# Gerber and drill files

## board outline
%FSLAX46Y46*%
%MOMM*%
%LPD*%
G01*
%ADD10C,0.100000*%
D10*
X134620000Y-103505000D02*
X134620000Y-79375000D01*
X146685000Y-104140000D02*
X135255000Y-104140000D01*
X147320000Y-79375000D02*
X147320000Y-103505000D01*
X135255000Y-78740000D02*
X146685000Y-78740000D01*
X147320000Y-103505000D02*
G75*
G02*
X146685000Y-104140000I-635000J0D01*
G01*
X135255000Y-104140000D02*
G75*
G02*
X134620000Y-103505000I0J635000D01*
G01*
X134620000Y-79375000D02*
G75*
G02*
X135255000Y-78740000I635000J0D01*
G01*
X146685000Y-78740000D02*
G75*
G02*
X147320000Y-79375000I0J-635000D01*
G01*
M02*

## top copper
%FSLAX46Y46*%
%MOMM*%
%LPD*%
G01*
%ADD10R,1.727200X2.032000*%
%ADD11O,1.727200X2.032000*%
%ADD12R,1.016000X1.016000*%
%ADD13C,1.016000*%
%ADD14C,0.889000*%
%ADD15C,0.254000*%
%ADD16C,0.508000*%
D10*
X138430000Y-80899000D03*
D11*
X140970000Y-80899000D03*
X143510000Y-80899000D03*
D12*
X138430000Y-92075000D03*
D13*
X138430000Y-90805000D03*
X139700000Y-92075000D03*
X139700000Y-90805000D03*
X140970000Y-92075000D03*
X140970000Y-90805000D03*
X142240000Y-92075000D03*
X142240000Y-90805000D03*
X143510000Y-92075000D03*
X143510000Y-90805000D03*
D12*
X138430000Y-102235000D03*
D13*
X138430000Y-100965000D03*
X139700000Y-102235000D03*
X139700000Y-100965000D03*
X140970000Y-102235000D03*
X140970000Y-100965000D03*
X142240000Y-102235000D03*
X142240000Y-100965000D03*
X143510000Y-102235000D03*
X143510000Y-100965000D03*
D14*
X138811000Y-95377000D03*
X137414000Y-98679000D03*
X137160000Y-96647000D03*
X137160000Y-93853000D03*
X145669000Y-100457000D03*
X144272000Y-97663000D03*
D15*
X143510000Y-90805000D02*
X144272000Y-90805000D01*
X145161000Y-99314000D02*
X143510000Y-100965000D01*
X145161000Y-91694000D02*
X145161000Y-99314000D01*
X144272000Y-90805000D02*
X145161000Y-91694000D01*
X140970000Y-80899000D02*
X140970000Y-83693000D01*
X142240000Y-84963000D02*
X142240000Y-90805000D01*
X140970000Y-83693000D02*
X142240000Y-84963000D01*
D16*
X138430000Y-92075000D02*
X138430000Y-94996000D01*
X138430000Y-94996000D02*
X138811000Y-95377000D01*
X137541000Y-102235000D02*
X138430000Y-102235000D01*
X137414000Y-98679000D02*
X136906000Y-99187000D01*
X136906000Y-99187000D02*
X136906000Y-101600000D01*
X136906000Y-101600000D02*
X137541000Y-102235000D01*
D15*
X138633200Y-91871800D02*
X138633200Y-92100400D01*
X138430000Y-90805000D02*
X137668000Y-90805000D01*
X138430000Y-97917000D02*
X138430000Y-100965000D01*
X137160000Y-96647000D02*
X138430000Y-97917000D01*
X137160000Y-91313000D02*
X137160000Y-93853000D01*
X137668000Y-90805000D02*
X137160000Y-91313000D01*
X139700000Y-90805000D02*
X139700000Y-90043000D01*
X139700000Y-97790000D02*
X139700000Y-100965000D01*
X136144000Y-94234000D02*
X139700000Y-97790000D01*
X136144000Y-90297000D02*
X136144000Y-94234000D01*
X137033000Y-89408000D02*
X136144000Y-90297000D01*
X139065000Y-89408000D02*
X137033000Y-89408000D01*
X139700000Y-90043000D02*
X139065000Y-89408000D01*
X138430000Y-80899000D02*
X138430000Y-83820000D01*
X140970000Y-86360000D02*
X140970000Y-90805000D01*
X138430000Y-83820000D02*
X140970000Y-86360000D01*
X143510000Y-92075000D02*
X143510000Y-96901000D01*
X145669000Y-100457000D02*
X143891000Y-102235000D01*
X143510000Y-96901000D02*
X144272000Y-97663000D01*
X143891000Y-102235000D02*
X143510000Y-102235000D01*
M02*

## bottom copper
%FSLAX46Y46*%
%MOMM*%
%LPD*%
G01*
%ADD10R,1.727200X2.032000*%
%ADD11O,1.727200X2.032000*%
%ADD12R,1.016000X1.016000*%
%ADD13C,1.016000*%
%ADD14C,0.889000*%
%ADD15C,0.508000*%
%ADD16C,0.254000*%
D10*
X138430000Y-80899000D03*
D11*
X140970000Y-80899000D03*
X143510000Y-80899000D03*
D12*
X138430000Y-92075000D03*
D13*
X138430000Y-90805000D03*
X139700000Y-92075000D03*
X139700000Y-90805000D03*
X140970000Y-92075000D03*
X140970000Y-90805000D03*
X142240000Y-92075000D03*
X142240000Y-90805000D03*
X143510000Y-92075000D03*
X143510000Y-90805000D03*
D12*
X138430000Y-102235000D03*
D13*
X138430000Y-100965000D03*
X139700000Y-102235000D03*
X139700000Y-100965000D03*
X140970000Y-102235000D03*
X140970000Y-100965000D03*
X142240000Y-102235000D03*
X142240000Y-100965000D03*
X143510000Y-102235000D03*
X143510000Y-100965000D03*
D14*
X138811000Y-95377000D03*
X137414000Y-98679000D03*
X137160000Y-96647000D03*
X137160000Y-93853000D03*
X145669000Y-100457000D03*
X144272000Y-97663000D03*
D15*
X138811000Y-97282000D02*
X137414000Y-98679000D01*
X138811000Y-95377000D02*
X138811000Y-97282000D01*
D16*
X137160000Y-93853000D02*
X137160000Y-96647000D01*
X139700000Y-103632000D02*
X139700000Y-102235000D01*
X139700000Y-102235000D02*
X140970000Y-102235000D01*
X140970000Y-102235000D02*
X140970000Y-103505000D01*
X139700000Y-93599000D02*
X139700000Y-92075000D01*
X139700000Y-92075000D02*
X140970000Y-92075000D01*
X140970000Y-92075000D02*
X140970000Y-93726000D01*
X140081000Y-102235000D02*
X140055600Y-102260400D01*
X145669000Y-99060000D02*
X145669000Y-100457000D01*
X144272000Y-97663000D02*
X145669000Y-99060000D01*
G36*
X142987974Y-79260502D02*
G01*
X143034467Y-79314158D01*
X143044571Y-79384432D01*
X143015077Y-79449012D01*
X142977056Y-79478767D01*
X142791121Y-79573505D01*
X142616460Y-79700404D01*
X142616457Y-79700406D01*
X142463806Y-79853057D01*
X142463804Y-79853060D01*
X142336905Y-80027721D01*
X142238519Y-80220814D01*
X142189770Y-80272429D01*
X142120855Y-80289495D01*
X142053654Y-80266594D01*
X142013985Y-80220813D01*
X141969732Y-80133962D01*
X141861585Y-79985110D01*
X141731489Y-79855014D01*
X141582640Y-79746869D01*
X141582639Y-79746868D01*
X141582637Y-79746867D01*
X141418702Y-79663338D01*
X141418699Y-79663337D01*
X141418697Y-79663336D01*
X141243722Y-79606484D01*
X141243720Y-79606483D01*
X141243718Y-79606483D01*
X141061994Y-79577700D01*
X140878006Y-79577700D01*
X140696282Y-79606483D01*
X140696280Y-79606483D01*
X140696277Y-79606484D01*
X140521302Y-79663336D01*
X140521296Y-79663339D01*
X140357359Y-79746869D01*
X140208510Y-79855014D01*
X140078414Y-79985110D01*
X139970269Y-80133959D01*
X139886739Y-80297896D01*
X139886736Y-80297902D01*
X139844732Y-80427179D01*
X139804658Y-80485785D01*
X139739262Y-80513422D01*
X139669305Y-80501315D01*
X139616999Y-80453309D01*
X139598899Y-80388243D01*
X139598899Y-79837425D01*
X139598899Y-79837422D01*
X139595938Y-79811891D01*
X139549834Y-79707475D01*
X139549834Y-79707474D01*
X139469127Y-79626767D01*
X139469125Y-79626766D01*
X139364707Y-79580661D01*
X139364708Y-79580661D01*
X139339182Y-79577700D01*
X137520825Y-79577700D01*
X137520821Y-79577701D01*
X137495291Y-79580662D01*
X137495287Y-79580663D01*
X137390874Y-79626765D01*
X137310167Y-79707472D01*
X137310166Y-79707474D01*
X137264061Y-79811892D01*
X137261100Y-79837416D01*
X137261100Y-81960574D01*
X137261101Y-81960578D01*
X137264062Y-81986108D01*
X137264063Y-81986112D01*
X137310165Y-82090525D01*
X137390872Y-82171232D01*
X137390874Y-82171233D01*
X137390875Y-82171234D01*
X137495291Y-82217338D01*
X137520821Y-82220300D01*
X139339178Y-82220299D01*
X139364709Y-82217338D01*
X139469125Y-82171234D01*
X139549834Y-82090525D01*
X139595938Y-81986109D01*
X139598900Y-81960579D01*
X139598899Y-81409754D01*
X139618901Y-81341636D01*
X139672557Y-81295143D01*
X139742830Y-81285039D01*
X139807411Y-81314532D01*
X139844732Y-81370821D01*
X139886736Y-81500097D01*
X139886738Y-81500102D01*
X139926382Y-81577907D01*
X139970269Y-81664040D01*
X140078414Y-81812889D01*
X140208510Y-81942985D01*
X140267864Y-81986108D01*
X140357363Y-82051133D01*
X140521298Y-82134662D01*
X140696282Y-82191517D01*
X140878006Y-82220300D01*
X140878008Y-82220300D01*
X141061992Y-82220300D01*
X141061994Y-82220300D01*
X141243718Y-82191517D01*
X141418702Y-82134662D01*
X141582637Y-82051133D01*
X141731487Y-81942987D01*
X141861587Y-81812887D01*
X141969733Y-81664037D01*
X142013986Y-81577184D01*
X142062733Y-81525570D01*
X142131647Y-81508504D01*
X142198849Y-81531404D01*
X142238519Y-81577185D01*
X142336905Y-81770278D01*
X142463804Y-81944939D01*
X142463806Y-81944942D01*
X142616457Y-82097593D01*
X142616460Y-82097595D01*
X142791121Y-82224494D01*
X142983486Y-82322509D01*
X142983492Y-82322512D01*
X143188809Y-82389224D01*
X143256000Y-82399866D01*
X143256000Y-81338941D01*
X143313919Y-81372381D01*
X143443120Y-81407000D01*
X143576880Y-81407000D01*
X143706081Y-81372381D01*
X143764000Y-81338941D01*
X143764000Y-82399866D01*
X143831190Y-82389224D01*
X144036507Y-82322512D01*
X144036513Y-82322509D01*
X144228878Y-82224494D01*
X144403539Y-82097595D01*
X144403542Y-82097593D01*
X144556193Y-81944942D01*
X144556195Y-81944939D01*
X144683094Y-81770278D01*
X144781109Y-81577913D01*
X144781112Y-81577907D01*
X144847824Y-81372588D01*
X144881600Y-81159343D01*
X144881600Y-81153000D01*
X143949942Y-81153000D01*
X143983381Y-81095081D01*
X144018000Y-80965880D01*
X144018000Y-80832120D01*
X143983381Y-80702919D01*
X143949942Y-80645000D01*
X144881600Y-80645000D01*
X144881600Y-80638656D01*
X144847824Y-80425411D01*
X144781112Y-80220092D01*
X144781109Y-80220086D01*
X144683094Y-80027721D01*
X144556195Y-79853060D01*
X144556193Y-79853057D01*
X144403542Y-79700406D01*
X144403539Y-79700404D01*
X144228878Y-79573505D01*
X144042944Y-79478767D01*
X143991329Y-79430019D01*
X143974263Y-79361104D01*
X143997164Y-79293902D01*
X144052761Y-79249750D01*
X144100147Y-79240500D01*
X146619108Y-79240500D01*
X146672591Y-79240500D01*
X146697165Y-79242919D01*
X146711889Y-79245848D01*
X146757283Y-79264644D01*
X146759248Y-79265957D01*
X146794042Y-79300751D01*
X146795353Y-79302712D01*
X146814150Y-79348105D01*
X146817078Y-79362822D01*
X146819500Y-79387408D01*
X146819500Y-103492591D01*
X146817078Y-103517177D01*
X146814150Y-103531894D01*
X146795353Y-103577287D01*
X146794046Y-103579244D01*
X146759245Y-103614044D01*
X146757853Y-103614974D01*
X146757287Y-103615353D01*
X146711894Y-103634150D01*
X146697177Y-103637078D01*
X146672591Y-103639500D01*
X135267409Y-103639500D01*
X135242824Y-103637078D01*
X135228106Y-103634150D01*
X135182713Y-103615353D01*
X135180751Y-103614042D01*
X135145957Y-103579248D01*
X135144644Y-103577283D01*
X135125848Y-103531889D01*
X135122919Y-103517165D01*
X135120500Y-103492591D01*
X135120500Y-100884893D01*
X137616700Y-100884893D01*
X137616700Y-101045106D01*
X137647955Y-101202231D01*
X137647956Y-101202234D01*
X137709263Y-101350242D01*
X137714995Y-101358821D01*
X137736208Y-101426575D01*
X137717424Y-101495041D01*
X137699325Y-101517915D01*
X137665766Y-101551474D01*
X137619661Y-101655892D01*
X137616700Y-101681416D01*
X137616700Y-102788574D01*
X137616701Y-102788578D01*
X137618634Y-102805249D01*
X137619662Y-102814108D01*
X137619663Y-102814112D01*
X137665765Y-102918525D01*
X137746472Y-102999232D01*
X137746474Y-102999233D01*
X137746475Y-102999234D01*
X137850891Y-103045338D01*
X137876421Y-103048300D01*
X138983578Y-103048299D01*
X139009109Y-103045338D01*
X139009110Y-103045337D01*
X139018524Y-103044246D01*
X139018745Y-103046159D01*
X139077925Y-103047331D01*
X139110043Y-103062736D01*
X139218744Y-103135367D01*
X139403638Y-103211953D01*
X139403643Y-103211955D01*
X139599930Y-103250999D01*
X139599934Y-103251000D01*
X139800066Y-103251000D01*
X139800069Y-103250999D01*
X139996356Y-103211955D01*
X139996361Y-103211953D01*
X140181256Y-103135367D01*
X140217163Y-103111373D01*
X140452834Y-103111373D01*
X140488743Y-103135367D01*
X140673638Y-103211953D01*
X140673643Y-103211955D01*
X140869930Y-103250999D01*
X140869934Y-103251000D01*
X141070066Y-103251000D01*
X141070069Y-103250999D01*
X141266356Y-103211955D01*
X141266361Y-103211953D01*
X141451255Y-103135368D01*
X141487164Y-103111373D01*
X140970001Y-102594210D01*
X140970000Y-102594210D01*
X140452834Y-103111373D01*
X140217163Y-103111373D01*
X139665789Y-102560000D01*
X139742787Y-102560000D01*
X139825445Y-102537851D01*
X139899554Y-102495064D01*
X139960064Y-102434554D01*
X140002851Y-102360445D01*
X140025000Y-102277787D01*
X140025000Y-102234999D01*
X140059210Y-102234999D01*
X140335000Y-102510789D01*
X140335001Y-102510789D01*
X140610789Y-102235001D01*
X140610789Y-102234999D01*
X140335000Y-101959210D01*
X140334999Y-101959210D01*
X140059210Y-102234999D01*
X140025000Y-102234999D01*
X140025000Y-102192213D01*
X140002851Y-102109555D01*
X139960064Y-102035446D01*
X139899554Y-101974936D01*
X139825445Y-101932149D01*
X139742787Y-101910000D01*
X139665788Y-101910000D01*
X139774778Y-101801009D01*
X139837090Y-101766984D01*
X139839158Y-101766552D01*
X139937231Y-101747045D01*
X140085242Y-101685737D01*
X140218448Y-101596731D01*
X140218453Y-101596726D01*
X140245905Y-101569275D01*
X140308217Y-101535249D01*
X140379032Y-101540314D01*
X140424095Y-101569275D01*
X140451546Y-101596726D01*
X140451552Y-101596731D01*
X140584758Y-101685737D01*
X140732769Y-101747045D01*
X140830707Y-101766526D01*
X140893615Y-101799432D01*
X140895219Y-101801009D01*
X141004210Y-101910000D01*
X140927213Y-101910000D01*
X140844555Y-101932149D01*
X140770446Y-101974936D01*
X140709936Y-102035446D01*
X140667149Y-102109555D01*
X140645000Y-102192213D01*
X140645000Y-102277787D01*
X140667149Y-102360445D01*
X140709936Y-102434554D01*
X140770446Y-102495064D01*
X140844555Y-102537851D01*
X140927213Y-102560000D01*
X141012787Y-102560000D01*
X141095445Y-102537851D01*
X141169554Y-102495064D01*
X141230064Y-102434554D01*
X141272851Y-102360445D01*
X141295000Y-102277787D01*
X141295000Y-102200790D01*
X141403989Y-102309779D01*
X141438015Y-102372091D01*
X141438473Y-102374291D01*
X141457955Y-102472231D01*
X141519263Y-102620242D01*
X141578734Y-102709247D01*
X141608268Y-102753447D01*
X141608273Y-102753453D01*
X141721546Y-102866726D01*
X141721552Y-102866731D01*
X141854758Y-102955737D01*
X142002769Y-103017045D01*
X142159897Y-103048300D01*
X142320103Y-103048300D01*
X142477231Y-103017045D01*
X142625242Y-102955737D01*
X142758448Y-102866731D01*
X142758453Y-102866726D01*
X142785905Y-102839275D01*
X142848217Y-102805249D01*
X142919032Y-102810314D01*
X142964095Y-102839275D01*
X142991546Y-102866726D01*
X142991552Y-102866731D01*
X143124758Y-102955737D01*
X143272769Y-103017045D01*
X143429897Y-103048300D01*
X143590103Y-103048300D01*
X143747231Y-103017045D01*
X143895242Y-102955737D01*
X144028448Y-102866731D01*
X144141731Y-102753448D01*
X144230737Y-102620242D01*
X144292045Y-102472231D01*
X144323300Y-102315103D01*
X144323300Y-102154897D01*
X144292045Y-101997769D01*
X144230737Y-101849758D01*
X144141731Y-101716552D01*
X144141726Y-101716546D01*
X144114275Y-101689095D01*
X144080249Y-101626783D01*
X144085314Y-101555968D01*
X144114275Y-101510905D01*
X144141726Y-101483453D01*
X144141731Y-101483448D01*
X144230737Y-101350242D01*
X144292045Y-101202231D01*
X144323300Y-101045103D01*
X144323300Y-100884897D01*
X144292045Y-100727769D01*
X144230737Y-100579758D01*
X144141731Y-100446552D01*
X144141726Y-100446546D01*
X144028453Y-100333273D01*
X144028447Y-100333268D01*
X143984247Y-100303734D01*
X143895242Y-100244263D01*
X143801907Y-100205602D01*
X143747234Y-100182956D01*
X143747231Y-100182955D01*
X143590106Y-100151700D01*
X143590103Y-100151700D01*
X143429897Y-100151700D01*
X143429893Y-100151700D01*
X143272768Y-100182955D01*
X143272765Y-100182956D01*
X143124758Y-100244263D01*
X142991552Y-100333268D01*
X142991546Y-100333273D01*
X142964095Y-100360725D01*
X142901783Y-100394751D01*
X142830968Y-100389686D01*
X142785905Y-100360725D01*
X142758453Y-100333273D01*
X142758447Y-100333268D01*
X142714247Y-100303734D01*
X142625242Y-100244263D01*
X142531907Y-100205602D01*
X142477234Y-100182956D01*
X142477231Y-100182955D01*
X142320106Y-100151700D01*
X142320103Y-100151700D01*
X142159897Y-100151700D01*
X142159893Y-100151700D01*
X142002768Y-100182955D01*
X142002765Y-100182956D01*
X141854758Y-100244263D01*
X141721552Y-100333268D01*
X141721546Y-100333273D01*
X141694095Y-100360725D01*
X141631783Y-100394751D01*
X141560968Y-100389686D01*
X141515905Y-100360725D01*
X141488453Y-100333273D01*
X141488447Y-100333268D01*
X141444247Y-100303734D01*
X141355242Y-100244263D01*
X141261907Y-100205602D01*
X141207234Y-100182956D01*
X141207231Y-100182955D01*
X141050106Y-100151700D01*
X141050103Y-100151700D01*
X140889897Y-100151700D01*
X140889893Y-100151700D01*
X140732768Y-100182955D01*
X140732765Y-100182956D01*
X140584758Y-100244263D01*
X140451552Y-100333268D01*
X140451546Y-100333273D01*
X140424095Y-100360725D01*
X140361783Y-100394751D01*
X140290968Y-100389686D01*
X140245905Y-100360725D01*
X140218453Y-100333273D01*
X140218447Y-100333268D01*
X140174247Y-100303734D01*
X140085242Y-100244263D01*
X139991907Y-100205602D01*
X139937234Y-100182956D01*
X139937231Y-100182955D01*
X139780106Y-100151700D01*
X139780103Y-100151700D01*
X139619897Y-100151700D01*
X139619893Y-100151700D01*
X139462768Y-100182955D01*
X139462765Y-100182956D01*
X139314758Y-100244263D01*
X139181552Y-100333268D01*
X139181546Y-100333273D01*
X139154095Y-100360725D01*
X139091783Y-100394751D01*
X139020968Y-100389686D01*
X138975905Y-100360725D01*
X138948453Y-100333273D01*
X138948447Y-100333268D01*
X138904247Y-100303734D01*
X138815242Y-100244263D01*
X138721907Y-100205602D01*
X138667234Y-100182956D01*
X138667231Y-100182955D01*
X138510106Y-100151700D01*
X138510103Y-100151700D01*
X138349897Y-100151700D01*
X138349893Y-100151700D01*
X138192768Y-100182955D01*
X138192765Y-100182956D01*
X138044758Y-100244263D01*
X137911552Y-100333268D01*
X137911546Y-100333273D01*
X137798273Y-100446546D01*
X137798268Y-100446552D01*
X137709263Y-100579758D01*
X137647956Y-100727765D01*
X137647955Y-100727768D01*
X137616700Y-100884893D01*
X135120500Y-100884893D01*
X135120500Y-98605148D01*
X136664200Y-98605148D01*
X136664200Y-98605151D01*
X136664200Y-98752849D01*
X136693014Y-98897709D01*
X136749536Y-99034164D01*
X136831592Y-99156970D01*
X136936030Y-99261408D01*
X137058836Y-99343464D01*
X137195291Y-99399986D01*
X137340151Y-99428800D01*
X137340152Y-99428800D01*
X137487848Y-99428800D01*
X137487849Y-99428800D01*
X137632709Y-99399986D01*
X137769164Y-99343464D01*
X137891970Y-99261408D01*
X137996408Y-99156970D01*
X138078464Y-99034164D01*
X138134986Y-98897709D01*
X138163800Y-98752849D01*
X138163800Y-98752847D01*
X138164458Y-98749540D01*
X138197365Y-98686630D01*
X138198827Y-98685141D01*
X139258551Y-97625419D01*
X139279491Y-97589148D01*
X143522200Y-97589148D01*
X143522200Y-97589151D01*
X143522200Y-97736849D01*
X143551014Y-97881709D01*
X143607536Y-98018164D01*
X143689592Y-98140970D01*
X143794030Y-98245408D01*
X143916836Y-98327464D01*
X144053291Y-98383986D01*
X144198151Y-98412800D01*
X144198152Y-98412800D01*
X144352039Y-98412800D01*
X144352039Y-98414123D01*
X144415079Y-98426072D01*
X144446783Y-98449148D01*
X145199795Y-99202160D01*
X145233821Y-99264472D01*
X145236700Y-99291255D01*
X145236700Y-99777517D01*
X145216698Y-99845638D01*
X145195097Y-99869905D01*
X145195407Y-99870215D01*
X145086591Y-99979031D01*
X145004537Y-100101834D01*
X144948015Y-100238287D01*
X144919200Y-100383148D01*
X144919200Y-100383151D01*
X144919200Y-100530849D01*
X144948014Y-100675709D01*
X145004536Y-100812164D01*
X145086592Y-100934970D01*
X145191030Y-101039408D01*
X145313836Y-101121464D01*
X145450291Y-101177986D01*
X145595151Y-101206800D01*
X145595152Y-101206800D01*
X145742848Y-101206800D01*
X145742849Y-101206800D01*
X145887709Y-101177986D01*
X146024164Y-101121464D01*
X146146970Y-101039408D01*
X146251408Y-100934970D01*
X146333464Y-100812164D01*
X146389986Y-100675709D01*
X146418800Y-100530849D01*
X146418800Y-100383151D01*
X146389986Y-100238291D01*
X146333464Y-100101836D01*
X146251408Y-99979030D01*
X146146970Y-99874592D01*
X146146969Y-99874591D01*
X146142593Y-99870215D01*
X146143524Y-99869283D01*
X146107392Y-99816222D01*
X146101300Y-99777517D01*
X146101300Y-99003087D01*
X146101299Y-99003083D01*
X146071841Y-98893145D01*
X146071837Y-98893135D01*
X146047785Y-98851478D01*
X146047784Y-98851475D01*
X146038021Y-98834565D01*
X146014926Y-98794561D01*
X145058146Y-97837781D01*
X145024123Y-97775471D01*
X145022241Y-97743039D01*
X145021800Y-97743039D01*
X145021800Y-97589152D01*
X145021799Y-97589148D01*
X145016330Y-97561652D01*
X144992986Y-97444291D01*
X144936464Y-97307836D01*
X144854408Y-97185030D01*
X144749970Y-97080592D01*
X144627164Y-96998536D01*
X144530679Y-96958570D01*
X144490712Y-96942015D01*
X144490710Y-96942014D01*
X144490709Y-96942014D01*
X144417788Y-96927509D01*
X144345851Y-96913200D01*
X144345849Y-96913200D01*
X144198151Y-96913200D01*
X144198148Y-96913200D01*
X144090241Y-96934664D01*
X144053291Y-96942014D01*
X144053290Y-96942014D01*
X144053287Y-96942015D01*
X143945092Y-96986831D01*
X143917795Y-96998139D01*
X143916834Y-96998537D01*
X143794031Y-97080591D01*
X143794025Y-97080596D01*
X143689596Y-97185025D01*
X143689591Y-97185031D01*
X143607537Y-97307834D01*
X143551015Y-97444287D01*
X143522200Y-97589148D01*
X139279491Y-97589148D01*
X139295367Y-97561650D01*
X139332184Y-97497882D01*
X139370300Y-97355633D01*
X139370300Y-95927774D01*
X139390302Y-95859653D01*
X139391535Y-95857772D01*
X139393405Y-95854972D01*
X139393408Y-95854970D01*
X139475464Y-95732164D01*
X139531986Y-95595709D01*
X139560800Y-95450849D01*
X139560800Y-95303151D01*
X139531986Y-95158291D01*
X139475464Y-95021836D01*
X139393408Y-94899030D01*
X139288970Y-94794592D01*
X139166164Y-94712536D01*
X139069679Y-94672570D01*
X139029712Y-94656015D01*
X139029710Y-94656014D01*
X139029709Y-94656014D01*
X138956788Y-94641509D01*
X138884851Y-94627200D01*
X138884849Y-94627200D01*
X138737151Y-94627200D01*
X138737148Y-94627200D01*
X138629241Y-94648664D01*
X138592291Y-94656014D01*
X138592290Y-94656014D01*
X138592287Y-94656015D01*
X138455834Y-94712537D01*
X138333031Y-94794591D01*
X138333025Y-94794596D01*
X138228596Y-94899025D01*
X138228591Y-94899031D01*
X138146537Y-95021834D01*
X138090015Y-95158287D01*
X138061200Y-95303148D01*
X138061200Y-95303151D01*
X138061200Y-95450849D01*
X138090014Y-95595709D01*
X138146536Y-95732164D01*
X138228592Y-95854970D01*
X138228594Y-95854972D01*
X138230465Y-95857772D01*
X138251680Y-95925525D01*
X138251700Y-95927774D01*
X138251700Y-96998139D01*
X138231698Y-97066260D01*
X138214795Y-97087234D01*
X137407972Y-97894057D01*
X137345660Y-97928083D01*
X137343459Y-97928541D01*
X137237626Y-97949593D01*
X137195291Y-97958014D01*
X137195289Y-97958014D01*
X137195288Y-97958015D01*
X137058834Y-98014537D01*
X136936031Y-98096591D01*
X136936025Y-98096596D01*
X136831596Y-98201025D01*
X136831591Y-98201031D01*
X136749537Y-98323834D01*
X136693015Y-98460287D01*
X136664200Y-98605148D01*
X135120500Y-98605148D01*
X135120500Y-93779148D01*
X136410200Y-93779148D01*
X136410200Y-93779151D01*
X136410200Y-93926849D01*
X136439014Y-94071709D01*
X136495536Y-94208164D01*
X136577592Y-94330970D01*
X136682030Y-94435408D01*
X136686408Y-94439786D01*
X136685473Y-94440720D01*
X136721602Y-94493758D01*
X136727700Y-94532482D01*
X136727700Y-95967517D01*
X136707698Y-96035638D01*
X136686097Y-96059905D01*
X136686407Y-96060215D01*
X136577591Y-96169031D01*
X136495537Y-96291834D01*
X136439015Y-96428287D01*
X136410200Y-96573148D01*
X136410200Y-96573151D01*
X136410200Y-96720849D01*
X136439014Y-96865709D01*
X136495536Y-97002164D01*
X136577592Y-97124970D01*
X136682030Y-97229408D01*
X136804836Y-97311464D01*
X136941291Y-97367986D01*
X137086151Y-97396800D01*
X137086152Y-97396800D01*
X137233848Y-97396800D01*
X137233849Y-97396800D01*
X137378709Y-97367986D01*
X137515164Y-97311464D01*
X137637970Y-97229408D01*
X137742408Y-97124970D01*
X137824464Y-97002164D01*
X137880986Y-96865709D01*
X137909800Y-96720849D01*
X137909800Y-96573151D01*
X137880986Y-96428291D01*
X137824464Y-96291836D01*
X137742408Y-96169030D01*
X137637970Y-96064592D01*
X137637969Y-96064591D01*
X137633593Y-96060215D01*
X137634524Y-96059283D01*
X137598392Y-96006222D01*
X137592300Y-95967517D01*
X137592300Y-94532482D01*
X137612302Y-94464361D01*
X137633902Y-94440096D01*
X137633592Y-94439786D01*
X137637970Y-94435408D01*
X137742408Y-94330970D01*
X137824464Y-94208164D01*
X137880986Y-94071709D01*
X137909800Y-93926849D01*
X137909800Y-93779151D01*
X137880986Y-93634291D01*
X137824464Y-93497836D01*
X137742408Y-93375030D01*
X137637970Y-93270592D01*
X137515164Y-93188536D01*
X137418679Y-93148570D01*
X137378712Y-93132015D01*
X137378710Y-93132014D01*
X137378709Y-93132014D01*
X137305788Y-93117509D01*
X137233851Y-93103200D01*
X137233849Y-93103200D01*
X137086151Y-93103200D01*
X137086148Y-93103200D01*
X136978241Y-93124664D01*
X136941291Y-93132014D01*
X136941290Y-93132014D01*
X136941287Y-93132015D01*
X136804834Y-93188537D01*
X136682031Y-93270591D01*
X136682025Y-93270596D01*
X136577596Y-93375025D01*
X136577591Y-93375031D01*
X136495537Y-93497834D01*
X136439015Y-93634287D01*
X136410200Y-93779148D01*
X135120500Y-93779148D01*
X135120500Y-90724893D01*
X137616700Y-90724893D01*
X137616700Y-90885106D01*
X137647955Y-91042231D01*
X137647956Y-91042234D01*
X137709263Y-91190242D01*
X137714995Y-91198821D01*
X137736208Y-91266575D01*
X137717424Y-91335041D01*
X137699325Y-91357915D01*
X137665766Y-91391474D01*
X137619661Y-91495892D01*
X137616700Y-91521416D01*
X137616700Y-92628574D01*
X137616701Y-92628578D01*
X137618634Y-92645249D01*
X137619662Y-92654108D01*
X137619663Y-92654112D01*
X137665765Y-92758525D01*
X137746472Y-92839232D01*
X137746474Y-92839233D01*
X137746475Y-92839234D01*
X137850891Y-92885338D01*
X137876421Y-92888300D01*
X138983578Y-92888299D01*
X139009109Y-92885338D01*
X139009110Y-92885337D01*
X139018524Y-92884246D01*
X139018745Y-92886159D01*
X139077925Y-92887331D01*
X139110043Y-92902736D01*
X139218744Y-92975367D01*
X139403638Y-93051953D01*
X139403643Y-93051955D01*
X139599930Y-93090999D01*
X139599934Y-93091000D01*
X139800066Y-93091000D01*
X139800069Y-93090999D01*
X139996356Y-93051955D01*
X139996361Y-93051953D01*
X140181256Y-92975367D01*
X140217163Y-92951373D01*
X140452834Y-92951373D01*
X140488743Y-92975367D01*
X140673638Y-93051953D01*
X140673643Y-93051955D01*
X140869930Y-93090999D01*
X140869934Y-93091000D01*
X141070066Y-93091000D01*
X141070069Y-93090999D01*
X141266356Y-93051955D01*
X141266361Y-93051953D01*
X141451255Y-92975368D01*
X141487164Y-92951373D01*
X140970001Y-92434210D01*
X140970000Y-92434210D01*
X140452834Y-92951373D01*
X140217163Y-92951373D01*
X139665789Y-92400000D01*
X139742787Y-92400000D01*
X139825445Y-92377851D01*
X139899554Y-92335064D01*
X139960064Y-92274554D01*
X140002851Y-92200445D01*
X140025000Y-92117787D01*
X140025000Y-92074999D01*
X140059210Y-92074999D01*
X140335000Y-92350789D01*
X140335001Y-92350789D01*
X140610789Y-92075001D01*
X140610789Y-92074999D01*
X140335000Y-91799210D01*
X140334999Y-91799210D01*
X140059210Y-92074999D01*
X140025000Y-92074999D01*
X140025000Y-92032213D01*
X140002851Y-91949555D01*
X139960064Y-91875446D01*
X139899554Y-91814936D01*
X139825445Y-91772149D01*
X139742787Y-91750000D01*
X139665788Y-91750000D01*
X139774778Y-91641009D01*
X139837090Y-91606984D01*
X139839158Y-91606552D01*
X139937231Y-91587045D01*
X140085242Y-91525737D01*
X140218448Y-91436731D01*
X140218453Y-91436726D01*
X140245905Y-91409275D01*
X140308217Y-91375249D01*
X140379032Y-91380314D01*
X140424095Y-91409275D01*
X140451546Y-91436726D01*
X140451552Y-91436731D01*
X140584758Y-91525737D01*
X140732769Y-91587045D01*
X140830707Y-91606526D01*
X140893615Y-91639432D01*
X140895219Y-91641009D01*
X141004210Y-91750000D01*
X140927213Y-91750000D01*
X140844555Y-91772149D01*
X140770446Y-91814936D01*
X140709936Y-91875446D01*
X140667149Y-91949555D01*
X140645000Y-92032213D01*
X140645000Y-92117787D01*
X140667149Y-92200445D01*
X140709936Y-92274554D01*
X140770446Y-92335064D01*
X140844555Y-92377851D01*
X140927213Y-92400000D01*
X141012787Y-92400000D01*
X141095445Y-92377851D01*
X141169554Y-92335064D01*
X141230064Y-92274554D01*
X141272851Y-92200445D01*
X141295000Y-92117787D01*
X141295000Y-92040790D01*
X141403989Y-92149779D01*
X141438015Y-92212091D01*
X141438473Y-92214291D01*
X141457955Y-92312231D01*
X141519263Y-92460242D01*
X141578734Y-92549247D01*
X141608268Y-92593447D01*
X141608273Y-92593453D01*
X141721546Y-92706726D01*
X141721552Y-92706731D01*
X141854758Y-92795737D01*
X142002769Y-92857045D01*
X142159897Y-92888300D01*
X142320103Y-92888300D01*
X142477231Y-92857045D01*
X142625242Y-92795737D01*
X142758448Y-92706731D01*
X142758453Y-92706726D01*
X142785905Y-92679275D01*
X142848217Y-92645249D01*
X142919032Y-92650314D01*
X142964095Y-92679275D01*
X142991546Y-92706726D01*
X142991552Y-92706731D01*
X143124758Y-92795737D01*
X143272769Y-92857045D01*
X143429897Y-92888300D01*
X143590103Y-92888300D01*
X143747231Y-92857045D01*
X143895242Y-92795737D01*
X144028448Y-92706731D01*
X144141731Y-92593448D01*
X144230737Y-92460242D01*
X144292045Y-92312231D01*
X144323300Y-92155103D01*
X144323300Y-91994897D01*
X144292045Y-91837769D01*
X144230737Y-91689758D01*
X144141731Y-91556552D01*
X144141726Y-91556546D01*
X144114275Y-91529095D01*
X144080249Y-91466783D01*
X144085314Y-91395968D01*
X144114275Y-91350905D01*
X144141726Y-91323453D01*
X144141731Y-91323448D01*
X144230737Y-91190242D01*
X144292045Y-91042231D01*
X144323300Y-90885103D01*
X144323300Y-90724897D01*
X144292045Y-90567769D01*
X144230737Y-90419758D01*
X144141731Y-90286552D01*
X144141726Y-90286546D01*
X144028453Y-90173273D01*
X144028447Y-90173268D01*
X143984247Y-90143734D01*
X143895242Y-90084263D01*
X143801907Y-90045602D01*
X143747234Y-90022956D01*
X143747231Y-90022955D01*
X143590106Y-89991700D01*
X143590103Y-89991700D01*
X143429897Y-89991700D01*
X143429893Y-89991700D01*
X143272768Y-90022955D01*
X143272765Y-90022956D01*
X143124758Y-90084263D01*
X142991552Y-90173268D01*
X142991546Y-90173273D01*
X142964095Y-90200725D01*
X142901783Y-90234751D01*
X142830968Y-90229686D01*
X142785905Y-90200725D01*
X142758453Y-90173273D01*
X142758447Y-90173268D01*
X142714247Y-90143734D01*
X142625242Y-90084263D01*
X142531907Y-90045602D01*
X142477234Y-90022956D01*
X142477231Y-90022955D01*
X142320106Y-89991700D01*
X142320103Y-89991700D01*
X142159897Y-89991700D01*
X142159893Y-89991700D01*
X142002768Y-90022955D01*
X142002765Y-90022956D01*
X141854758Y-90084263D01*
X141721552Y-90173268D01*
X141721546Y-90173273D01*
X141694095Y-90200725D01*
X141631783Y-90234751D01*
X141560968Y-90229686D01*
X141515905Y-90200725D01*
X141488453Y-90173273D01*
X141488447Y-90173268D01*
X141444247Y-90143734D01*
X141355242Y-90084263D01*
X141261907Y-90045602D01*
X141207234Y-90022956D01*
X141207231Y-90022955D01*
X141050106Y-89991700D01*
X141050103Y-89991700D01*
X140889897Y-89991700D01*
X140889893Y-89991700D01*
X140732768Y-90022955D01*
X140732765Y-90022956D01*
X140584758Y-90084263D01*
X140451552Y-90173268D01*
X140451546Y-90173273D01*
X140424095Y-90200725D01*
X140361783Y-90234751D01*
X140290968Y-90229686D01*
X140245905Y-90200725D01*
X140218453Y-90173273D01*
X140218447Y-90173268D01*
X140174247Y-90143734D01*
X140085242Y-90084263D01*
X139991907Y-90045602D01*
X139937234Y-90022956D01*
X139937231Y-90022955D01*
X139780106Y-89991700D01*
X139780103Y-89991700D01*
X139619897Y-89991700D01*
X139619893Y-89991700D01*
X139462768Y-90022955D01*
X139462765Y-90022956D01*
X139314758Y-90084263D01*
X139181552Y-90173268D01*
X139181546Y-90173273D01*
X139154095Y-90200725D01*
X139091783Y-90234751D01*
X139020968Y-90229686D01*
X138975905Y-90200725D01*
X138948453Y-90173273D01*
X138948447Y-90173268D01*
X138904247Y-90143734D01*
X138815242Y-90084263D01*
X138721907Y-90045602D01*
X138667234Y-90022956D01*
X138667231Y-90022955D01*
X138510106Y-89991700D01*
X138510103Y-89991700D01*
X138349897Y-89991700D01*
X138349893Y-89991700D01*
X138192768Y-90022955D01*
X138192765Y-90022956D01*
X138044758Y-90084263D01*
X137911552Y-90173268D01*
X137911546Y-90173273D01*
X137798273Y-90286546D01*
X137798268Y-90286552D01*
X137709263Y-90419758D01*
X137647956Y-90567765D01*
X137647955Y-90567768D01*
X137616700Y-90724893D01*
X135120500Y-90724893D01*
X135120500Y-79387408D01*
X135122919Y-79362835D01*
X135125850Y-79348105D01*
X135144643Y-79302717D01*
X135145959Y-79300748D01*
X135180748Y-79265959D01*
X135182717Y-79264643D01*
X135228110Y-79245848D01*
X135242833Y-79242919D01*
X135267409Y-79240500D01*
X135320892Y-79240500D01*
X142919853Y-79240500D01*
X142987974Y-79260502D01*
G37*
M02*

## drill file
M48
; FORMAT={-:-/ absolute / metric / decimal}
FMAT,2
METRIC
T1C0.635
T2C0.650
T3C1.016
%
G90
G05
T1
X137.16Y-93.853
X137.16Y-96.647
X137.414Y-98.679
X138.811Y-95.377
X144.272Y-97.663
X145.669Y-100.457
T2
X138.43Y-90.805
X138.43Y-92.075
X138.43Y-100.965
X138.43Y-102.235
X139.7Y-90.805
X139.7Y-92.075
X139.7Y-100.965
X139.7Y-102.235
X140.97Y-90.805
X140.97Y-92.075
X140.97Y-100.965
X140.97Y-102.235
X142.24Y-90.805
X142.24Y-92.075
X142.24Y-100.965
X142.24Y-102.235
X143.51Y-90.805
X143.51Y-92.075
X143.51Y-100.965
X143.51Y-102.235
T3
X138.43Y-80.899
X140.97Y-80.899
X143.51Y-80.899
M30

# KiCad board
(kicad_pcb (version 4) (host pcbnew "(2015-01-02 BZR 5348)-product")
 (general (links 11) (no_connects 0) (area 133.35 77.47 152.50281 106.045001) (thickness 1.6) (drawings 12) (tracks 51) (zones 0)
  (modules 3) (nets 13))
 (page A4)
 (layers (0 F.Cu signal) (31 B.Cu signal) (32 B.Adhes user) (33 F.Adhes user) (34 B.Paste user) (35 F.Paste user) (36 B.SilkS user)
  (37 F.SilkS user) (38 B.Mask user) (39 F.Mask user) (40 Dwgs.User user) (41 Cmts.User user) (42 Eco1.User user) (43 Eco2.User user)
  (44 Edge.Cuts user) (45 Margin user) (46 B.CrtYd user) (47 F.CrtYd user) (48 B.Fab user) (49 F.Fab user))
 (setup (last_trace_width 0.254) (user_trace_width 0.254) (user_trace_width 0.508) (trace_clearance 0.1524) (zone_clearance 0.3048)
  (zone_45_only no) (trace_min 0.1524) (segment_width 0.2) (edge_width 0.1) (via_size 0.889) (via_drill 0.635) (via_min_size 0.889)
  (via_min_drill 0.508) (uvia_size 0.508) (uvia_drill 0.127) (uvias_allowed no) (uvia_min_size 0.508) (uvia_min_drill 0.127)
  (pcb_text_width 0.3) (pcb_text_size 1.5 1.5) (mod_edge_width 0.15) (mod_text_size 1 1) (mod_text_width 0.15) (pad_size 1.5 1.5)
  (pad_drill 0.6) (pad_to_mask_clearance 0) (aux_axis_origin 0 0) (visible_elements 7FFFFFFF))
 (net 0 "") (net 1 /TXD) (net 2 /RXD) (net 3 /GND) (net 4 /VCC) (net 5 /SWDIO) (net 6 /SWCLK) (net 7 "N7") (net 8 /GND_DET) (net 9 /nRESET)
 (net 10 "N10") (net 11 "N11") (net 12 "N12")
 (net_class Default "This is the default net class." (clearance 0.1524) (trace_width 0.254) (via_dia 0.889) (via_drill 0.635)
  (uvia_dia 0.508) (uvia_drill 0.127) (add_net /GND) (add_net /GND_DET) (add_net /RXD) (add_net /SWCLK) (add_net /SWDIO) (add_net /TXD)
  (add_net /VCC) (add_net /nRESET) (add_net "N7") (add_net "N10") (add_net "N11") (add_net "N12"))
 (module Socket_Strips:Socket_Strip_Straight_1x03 (layer F.Cu) (at 140.97 80.899 180)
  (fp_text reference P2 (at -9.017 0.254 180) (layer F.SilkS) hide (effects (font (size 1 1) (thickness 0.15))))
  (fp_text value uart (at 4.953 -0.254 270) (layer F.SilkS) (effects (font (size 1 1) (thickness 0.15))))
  (pad 1 thru_hole rect (at 2.54 0) (size 1.7272 2.032) (drill 1.016) (layers *.Cu *.Mask F.SilkS) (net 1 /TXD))
  (pad 2 thru_hole oval (at 0 0) (size 1.7272 2.032) (drill 1.016) (layers *.Cu *.Mask F.SilkS) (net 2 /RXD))
  (pad 3 thru_hole oval (at -2.54 0) (size 1.7272 2.032) (drill 1.016) (layers *.Cu *.Mask F.SilkS) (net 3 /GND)))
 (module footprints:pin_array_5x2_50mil (layer F.Cu) (at 139.7 91.44)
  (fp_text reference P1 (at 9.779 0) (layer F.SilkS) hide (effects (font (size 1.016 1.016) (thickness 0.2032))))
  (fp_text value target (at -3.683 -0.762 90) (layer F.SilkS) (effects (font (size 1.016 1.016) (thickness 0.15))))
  (pad 1 thru_hole rect (at -1.27 0.635) (size 1.016 1.016) (drill 0.65) (layers *.Cu *.Mask F.SilkS) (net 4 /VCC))
  (pad 2 thru_hole circle (at -1.27 -0.635) (size 1.016 1.016) (drill 0.65) (layers *.Cu *.Mask F.SilkS) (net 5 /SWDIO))
  (pad 3 thru_hole circle (at 0 0.635) (size 1.016 1.016) (drill 0.65) (layers *.Cu *.Mask F.SilkS) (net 3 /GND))
  (pad 4 thru_hole circle (at 0 -0.635) (size 1.016 1.016) (drill 0.65) (layers *.Cu *.Mask F.SilkS) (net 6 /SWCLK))
  (pad 5 thru_hole circle (at 1.27 0.635) (size 1.016 1.016) (drill 0.65) (layers *.Cu *.Mask F.SilkS) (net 3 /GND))
  (pad 6 thru_hole circle (at 1.27 -0.635) (size 1.016 1.016) (drill 0.65) (layers *.Cu *.Mask F.SilkS) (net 1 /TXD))
  (pad 7 thru_hole circle (at 2.54 0.635) (size 1.016 1.016) (drill 0.65) (layers *.Cu *.Mask F.SilkS) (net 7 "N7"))
  (pad 8 thru_hole circle (at 2.54 -0.635) (size 1.016 1.016) (drill 0.65) (layers *.Cu *.Mask F.SilkS) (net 2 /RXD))
  (pad 9 thru_hole circle (at 3.81 0.635) (size 1.016 1.016) (drill 0.65) (layers *.Cu *.Mask F.SilkS) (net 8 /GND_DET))
  (pad 10 thru_hole circle (at 3.81 -0.635) (size 1.016 1.016) (drill 0.65) (layers *.Cu *.Mask F.SilkS) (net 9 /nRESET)))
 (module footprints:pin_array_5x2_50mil (layer F.Cu) (at 139.7 101.6)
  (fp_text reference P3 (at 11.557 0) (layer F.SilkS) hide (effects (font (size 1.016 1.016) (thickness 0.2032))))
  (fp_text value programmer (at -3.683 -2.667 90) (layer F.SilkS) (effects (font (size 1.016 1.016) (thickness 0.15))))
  (pad 1 thru_hole rect (at -1.27 0.635) (size 1.016 1.016) (drill 0.65) (layers *.Cu *.Mask F.SilkS) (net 4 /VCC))
  (pad 2 thru_hole circle (at -1.27 -0.635) (size 1.016 1.016) (drill 0.65) (layers *.Cu *.Mask F.SilkS) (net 5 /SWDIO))
  (pad 3 thru_hole circle (at 0 0.635) (size 1.016 1.016) (drill 0.65) (layers *.Cu *.Mask F.SilkS) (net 3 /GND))
  (pad 4 thru_hole circle (at 0 -0.635) (size 1.016 1.016) (drill 0.65) (layers *.Cu *.Mask F.SilkS) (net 6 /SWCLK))
  (pad 5 thru_hole circle (at 1.27 0.635) (size 1.016 1.016) (drill 0.65) (layers *.Cu *.Mask F.SilkS) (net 3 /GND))
  (pad 6 thru_hole circle (at 1.27 -0.635) (size 1.016 1.016) (drill 0.65) (layers *.Cu *.Mask F.SilkS) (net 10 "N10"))
  (pad 7 thru_hole circle (at 2.54 0.635) (size 1.016 1.016) (drill 0.65) (layers *.Cu *.Mask F.SilkS) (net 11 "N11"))
  (pad 8 thru_hole circle (at 2.54 -0.635) (size 1.016 1.016) (drill 0.65) (layers *.Cu *.Mask F.SilkS) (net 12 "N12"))
  (pad 9 thru_hole circle (at 3.81 0.635) (size 1.016 1.016) (drill 0.65) (layers *.Cu *.Mask F.SilkS) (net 8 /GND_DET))
  (pad 10 thru_hole circle (at 3.81 -0.635) (size 1.016 1.016) (drill 0.65) (layers *.Cu *.Mask F.SilkS) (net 9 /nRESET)))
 (gr_line (start 134.62 103.505) (end 134.62 79.375) (angle 90) (layer Edge.Cuts) (width 0.1))
 (gr_line (start 146.685 104.14) (end 135.255 104.14) (angle 90) (layer Edge.Cuts) (width 0.1))
 (gr_line (start 147.32 79.375) (end 147.32 103.505) (angle 90) (layer Edge.Cuts) (width 0.1))
 (gr_line (start 135.255 78.74) (end 146.685 78.74) (angle 90) (layer Edge.Cuts) (width 0.1))
 (gr_arc (start 146.685 103.505) (end 147.32 103.505) (angle 90) (layer Edge.Cuts) (width 0.1))
 (gr_arc (start 135.255 103.505) (end 135.255 104.14) (angle 90) (layer Edge.Cuts) (width 0.1))
 (gr_arc (start 135.255 79.375) (end 134.62 79.375) (angle 90) (layer Edge.Cuts) (width 0.1))
 (gr_arc (start 146.685 79.375) (end 146.685 78.74) (angle 90) (layer Edge.Cuts) (width 0.1))
 (segment (start 143.51 90.805) (end 144.272 90.805) (width 0.254) (layer F.Cu) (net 9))
 (segment (start 145.161 99.314) (end 143.51 100.965) (width 0.254) (layer F.Cu) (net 9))
 (segment (start 145.161 91.694) (end 145.161 99.314) (width 0.254) (layer F.Cu) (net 9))
 (segment (start 144.272 90.805) (end 145.161 91.694) (width 0.254) (layer F.Cu) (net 9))
 (segment (start 140.97 80.899) (end 140.97 83.693) (width 0.254) (layer F.Cu) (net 2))
 (segment (start 142.24 84.963) (end 142.24 90.805) (width 0.254) (layer F.Cu) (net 2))
 (segment (start 140.97 83.693) (end 142.24 84.963) (width 0.254) (layer F.Cu) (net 2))
 (segment (start 138.43 92.075) (end 138.43 94.996) (width 0.508) (layer F.Cu) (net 4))
 (segment (start 138.811 97.282) (end 137.414 98.679) (width 0.508) (layer B.Cu) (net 4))
 (segment (start 138.811 95.377) (end 138.811 97.282) (width 0.508) (layer B.Cu) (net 4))
 (via (at 138.811 95.377) (size 0.889) (layers F.Cu B.Cu) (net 4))
 (segment (start 138.43 94.996) (end 138.811 95.377) (width 0.508) (layer F.Cu) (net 4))
 (segment (start 137.541 102.235) (end 138.43 102.235) (width 0.508) (layer F.Cu) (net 4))
 (via (at 137.414 98.679) (size 0.889) (layers F.Cu B.Cu) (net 4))
 (segment (start 137.414 98.679) (end 136.906 99.187) (width 0.508) (layer F.Cu) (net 4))
 (segment (start 136.906 99.187) (end 136.906 101.6) (width 0.508) (layer F.Cu) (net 4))
 (segment (start 136.906 101.6) (end 137.541 102.235) (width 0.508) (layer F.Cu) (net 4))
 (segment (start 138.6332 91.8718) (end 138.6332 92.1004) (width 0.254) (layer F.Cu) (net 4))
 (segment (start 138.43 90.805) (end 137.668 90.805) (width 0.254) (layer F.Cu) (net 5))
 (segment (start 138.43 97.917) (end 138.43 100.965) (width 0.254) (layer F.Cu) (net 5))
 (segment (start 137.16 96.647) (end 138.43 97.917) (width 0.254) (layer F.Cu) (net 5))
 (via (at 137.16 96.647) (size 0.889) (layers F.Cu B.Cu) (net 5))
 (segment (start 137.16 93.853) (end 137.16 96.647) (width 0.254) (layer B.Cu) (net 5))
 (via (at 137.16 93.853) (size 0.889) (layers F.Cu B.Cu) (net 5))
 (segment (start 137.16 91.313) (end 137.16 93.853) (width 0.254) (layer F.Cu) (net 5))
 (segment (start 137.668 90.805) (end 137.16 91.313) (width 0.254) (layer F.Cu) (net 5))
 (segment (start 139.7 103.632) (end 139.7 102.235) (width 0.254) (layer B.Cu) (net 3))
 (segment (start 139.7 102.235) (end 140.97 102.235) (width 0.254) (layer B.Cu) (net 3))
 (segment (start 140.97 102.235) (end 140.97 103.505) (width 0.254) (layer B.Cu) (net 3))
 (segment (start 139.7 93.599) (end 139.7 92.075) (width 0.254) (layer B.Cu) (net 3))
 (segment (start 139.7 92.075) (end 140.97 92.075) (width 0.254) (layer B.Cu) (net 3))
 (segment (start 140.97 92.075) (end 140.97 93.726) (width 0.254) (layer B.Cu) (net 3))
 (segment (start 140.081 102.235) (end 140.0556 102.2604) (width 0.254) (layer B.Cu) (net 3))
 (segment (start 139.7 90.805) (end 139.7 90.043) (width 0.254) (layer F.Cu) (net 6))
 (segment (start 139.7 97.79) (end 139.7 100.965) (width 0.254) (layer F.Cu) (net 6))
 (segment (start 136.144 94.234) (end 139.7 97.79) (width 0.254) (layer F.Cu) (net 6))
 (segment (start 136.144 90.297) (end 136.144 94.234) (width 0.254) (layer F.Cu) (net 6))
 (segment (start 137.033 89.408) (end 136.144 90.297) (width 0.254) (layer F.Cu) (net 6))
 (segment (start 139.065 89.408) (end 137.033 89.408) (width 0.254) (layer F.Cu) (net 6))
 (segment (start 139.7 90.043) (end 139.065 89.408) (width 0.254) (layer F.Cu) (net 6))
 (segment (start 138.43 80.899) (end 138.43 83.82) (width 0.254) (layer F.Cu) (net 1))
 (segment (start 140.97 86.36) (end 140.97 90.805) (width 0.254) (layer F.Cu) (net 1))
 (segment (start 138.43 83.82) (end 140.97 86.36) (width 0.254) (layer F.Cu) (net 1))
 (segment (start 143.51 92.075) (end 143.51 96.901) (width 0.254) (layer F.Cu) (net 8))
 (segment (start 145.669 100.457) (end 143.891 102.235) (width 0.254) (layer F.Cu) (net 8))
 (via (at 145.669 100.457) (size 0.889) (layers F.Cu B.Cu) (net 8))
 (segment (start 145.669 99.06) (end 145.669 100.457) (width 0.254) (layer B.Cu) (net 8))
 (segment (start 144.272 97.663) (end 145.669 99.06) (width 0.254) (layer B.Cu) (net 8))
 (via (at 144.272 97.663) (size 0.889) (layers F.Cu B.Cu) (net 8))
 (segment (start 143.51 96.901) (end 144.272 97.663) (width 0.254) (layer F.Cu) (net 8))
 (segment (start 143.891 102.235) (end 143.51 102.235) (width 0.254) (layer F.Cu) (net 8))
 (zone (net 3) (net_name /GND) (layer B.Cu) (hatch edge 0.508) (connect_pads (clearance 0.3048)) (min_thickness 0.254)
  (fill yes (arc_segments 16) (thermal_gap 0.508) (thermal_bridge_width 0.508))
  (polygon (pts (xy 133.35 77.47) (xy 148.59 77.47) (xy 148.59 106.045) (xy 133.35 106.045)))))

